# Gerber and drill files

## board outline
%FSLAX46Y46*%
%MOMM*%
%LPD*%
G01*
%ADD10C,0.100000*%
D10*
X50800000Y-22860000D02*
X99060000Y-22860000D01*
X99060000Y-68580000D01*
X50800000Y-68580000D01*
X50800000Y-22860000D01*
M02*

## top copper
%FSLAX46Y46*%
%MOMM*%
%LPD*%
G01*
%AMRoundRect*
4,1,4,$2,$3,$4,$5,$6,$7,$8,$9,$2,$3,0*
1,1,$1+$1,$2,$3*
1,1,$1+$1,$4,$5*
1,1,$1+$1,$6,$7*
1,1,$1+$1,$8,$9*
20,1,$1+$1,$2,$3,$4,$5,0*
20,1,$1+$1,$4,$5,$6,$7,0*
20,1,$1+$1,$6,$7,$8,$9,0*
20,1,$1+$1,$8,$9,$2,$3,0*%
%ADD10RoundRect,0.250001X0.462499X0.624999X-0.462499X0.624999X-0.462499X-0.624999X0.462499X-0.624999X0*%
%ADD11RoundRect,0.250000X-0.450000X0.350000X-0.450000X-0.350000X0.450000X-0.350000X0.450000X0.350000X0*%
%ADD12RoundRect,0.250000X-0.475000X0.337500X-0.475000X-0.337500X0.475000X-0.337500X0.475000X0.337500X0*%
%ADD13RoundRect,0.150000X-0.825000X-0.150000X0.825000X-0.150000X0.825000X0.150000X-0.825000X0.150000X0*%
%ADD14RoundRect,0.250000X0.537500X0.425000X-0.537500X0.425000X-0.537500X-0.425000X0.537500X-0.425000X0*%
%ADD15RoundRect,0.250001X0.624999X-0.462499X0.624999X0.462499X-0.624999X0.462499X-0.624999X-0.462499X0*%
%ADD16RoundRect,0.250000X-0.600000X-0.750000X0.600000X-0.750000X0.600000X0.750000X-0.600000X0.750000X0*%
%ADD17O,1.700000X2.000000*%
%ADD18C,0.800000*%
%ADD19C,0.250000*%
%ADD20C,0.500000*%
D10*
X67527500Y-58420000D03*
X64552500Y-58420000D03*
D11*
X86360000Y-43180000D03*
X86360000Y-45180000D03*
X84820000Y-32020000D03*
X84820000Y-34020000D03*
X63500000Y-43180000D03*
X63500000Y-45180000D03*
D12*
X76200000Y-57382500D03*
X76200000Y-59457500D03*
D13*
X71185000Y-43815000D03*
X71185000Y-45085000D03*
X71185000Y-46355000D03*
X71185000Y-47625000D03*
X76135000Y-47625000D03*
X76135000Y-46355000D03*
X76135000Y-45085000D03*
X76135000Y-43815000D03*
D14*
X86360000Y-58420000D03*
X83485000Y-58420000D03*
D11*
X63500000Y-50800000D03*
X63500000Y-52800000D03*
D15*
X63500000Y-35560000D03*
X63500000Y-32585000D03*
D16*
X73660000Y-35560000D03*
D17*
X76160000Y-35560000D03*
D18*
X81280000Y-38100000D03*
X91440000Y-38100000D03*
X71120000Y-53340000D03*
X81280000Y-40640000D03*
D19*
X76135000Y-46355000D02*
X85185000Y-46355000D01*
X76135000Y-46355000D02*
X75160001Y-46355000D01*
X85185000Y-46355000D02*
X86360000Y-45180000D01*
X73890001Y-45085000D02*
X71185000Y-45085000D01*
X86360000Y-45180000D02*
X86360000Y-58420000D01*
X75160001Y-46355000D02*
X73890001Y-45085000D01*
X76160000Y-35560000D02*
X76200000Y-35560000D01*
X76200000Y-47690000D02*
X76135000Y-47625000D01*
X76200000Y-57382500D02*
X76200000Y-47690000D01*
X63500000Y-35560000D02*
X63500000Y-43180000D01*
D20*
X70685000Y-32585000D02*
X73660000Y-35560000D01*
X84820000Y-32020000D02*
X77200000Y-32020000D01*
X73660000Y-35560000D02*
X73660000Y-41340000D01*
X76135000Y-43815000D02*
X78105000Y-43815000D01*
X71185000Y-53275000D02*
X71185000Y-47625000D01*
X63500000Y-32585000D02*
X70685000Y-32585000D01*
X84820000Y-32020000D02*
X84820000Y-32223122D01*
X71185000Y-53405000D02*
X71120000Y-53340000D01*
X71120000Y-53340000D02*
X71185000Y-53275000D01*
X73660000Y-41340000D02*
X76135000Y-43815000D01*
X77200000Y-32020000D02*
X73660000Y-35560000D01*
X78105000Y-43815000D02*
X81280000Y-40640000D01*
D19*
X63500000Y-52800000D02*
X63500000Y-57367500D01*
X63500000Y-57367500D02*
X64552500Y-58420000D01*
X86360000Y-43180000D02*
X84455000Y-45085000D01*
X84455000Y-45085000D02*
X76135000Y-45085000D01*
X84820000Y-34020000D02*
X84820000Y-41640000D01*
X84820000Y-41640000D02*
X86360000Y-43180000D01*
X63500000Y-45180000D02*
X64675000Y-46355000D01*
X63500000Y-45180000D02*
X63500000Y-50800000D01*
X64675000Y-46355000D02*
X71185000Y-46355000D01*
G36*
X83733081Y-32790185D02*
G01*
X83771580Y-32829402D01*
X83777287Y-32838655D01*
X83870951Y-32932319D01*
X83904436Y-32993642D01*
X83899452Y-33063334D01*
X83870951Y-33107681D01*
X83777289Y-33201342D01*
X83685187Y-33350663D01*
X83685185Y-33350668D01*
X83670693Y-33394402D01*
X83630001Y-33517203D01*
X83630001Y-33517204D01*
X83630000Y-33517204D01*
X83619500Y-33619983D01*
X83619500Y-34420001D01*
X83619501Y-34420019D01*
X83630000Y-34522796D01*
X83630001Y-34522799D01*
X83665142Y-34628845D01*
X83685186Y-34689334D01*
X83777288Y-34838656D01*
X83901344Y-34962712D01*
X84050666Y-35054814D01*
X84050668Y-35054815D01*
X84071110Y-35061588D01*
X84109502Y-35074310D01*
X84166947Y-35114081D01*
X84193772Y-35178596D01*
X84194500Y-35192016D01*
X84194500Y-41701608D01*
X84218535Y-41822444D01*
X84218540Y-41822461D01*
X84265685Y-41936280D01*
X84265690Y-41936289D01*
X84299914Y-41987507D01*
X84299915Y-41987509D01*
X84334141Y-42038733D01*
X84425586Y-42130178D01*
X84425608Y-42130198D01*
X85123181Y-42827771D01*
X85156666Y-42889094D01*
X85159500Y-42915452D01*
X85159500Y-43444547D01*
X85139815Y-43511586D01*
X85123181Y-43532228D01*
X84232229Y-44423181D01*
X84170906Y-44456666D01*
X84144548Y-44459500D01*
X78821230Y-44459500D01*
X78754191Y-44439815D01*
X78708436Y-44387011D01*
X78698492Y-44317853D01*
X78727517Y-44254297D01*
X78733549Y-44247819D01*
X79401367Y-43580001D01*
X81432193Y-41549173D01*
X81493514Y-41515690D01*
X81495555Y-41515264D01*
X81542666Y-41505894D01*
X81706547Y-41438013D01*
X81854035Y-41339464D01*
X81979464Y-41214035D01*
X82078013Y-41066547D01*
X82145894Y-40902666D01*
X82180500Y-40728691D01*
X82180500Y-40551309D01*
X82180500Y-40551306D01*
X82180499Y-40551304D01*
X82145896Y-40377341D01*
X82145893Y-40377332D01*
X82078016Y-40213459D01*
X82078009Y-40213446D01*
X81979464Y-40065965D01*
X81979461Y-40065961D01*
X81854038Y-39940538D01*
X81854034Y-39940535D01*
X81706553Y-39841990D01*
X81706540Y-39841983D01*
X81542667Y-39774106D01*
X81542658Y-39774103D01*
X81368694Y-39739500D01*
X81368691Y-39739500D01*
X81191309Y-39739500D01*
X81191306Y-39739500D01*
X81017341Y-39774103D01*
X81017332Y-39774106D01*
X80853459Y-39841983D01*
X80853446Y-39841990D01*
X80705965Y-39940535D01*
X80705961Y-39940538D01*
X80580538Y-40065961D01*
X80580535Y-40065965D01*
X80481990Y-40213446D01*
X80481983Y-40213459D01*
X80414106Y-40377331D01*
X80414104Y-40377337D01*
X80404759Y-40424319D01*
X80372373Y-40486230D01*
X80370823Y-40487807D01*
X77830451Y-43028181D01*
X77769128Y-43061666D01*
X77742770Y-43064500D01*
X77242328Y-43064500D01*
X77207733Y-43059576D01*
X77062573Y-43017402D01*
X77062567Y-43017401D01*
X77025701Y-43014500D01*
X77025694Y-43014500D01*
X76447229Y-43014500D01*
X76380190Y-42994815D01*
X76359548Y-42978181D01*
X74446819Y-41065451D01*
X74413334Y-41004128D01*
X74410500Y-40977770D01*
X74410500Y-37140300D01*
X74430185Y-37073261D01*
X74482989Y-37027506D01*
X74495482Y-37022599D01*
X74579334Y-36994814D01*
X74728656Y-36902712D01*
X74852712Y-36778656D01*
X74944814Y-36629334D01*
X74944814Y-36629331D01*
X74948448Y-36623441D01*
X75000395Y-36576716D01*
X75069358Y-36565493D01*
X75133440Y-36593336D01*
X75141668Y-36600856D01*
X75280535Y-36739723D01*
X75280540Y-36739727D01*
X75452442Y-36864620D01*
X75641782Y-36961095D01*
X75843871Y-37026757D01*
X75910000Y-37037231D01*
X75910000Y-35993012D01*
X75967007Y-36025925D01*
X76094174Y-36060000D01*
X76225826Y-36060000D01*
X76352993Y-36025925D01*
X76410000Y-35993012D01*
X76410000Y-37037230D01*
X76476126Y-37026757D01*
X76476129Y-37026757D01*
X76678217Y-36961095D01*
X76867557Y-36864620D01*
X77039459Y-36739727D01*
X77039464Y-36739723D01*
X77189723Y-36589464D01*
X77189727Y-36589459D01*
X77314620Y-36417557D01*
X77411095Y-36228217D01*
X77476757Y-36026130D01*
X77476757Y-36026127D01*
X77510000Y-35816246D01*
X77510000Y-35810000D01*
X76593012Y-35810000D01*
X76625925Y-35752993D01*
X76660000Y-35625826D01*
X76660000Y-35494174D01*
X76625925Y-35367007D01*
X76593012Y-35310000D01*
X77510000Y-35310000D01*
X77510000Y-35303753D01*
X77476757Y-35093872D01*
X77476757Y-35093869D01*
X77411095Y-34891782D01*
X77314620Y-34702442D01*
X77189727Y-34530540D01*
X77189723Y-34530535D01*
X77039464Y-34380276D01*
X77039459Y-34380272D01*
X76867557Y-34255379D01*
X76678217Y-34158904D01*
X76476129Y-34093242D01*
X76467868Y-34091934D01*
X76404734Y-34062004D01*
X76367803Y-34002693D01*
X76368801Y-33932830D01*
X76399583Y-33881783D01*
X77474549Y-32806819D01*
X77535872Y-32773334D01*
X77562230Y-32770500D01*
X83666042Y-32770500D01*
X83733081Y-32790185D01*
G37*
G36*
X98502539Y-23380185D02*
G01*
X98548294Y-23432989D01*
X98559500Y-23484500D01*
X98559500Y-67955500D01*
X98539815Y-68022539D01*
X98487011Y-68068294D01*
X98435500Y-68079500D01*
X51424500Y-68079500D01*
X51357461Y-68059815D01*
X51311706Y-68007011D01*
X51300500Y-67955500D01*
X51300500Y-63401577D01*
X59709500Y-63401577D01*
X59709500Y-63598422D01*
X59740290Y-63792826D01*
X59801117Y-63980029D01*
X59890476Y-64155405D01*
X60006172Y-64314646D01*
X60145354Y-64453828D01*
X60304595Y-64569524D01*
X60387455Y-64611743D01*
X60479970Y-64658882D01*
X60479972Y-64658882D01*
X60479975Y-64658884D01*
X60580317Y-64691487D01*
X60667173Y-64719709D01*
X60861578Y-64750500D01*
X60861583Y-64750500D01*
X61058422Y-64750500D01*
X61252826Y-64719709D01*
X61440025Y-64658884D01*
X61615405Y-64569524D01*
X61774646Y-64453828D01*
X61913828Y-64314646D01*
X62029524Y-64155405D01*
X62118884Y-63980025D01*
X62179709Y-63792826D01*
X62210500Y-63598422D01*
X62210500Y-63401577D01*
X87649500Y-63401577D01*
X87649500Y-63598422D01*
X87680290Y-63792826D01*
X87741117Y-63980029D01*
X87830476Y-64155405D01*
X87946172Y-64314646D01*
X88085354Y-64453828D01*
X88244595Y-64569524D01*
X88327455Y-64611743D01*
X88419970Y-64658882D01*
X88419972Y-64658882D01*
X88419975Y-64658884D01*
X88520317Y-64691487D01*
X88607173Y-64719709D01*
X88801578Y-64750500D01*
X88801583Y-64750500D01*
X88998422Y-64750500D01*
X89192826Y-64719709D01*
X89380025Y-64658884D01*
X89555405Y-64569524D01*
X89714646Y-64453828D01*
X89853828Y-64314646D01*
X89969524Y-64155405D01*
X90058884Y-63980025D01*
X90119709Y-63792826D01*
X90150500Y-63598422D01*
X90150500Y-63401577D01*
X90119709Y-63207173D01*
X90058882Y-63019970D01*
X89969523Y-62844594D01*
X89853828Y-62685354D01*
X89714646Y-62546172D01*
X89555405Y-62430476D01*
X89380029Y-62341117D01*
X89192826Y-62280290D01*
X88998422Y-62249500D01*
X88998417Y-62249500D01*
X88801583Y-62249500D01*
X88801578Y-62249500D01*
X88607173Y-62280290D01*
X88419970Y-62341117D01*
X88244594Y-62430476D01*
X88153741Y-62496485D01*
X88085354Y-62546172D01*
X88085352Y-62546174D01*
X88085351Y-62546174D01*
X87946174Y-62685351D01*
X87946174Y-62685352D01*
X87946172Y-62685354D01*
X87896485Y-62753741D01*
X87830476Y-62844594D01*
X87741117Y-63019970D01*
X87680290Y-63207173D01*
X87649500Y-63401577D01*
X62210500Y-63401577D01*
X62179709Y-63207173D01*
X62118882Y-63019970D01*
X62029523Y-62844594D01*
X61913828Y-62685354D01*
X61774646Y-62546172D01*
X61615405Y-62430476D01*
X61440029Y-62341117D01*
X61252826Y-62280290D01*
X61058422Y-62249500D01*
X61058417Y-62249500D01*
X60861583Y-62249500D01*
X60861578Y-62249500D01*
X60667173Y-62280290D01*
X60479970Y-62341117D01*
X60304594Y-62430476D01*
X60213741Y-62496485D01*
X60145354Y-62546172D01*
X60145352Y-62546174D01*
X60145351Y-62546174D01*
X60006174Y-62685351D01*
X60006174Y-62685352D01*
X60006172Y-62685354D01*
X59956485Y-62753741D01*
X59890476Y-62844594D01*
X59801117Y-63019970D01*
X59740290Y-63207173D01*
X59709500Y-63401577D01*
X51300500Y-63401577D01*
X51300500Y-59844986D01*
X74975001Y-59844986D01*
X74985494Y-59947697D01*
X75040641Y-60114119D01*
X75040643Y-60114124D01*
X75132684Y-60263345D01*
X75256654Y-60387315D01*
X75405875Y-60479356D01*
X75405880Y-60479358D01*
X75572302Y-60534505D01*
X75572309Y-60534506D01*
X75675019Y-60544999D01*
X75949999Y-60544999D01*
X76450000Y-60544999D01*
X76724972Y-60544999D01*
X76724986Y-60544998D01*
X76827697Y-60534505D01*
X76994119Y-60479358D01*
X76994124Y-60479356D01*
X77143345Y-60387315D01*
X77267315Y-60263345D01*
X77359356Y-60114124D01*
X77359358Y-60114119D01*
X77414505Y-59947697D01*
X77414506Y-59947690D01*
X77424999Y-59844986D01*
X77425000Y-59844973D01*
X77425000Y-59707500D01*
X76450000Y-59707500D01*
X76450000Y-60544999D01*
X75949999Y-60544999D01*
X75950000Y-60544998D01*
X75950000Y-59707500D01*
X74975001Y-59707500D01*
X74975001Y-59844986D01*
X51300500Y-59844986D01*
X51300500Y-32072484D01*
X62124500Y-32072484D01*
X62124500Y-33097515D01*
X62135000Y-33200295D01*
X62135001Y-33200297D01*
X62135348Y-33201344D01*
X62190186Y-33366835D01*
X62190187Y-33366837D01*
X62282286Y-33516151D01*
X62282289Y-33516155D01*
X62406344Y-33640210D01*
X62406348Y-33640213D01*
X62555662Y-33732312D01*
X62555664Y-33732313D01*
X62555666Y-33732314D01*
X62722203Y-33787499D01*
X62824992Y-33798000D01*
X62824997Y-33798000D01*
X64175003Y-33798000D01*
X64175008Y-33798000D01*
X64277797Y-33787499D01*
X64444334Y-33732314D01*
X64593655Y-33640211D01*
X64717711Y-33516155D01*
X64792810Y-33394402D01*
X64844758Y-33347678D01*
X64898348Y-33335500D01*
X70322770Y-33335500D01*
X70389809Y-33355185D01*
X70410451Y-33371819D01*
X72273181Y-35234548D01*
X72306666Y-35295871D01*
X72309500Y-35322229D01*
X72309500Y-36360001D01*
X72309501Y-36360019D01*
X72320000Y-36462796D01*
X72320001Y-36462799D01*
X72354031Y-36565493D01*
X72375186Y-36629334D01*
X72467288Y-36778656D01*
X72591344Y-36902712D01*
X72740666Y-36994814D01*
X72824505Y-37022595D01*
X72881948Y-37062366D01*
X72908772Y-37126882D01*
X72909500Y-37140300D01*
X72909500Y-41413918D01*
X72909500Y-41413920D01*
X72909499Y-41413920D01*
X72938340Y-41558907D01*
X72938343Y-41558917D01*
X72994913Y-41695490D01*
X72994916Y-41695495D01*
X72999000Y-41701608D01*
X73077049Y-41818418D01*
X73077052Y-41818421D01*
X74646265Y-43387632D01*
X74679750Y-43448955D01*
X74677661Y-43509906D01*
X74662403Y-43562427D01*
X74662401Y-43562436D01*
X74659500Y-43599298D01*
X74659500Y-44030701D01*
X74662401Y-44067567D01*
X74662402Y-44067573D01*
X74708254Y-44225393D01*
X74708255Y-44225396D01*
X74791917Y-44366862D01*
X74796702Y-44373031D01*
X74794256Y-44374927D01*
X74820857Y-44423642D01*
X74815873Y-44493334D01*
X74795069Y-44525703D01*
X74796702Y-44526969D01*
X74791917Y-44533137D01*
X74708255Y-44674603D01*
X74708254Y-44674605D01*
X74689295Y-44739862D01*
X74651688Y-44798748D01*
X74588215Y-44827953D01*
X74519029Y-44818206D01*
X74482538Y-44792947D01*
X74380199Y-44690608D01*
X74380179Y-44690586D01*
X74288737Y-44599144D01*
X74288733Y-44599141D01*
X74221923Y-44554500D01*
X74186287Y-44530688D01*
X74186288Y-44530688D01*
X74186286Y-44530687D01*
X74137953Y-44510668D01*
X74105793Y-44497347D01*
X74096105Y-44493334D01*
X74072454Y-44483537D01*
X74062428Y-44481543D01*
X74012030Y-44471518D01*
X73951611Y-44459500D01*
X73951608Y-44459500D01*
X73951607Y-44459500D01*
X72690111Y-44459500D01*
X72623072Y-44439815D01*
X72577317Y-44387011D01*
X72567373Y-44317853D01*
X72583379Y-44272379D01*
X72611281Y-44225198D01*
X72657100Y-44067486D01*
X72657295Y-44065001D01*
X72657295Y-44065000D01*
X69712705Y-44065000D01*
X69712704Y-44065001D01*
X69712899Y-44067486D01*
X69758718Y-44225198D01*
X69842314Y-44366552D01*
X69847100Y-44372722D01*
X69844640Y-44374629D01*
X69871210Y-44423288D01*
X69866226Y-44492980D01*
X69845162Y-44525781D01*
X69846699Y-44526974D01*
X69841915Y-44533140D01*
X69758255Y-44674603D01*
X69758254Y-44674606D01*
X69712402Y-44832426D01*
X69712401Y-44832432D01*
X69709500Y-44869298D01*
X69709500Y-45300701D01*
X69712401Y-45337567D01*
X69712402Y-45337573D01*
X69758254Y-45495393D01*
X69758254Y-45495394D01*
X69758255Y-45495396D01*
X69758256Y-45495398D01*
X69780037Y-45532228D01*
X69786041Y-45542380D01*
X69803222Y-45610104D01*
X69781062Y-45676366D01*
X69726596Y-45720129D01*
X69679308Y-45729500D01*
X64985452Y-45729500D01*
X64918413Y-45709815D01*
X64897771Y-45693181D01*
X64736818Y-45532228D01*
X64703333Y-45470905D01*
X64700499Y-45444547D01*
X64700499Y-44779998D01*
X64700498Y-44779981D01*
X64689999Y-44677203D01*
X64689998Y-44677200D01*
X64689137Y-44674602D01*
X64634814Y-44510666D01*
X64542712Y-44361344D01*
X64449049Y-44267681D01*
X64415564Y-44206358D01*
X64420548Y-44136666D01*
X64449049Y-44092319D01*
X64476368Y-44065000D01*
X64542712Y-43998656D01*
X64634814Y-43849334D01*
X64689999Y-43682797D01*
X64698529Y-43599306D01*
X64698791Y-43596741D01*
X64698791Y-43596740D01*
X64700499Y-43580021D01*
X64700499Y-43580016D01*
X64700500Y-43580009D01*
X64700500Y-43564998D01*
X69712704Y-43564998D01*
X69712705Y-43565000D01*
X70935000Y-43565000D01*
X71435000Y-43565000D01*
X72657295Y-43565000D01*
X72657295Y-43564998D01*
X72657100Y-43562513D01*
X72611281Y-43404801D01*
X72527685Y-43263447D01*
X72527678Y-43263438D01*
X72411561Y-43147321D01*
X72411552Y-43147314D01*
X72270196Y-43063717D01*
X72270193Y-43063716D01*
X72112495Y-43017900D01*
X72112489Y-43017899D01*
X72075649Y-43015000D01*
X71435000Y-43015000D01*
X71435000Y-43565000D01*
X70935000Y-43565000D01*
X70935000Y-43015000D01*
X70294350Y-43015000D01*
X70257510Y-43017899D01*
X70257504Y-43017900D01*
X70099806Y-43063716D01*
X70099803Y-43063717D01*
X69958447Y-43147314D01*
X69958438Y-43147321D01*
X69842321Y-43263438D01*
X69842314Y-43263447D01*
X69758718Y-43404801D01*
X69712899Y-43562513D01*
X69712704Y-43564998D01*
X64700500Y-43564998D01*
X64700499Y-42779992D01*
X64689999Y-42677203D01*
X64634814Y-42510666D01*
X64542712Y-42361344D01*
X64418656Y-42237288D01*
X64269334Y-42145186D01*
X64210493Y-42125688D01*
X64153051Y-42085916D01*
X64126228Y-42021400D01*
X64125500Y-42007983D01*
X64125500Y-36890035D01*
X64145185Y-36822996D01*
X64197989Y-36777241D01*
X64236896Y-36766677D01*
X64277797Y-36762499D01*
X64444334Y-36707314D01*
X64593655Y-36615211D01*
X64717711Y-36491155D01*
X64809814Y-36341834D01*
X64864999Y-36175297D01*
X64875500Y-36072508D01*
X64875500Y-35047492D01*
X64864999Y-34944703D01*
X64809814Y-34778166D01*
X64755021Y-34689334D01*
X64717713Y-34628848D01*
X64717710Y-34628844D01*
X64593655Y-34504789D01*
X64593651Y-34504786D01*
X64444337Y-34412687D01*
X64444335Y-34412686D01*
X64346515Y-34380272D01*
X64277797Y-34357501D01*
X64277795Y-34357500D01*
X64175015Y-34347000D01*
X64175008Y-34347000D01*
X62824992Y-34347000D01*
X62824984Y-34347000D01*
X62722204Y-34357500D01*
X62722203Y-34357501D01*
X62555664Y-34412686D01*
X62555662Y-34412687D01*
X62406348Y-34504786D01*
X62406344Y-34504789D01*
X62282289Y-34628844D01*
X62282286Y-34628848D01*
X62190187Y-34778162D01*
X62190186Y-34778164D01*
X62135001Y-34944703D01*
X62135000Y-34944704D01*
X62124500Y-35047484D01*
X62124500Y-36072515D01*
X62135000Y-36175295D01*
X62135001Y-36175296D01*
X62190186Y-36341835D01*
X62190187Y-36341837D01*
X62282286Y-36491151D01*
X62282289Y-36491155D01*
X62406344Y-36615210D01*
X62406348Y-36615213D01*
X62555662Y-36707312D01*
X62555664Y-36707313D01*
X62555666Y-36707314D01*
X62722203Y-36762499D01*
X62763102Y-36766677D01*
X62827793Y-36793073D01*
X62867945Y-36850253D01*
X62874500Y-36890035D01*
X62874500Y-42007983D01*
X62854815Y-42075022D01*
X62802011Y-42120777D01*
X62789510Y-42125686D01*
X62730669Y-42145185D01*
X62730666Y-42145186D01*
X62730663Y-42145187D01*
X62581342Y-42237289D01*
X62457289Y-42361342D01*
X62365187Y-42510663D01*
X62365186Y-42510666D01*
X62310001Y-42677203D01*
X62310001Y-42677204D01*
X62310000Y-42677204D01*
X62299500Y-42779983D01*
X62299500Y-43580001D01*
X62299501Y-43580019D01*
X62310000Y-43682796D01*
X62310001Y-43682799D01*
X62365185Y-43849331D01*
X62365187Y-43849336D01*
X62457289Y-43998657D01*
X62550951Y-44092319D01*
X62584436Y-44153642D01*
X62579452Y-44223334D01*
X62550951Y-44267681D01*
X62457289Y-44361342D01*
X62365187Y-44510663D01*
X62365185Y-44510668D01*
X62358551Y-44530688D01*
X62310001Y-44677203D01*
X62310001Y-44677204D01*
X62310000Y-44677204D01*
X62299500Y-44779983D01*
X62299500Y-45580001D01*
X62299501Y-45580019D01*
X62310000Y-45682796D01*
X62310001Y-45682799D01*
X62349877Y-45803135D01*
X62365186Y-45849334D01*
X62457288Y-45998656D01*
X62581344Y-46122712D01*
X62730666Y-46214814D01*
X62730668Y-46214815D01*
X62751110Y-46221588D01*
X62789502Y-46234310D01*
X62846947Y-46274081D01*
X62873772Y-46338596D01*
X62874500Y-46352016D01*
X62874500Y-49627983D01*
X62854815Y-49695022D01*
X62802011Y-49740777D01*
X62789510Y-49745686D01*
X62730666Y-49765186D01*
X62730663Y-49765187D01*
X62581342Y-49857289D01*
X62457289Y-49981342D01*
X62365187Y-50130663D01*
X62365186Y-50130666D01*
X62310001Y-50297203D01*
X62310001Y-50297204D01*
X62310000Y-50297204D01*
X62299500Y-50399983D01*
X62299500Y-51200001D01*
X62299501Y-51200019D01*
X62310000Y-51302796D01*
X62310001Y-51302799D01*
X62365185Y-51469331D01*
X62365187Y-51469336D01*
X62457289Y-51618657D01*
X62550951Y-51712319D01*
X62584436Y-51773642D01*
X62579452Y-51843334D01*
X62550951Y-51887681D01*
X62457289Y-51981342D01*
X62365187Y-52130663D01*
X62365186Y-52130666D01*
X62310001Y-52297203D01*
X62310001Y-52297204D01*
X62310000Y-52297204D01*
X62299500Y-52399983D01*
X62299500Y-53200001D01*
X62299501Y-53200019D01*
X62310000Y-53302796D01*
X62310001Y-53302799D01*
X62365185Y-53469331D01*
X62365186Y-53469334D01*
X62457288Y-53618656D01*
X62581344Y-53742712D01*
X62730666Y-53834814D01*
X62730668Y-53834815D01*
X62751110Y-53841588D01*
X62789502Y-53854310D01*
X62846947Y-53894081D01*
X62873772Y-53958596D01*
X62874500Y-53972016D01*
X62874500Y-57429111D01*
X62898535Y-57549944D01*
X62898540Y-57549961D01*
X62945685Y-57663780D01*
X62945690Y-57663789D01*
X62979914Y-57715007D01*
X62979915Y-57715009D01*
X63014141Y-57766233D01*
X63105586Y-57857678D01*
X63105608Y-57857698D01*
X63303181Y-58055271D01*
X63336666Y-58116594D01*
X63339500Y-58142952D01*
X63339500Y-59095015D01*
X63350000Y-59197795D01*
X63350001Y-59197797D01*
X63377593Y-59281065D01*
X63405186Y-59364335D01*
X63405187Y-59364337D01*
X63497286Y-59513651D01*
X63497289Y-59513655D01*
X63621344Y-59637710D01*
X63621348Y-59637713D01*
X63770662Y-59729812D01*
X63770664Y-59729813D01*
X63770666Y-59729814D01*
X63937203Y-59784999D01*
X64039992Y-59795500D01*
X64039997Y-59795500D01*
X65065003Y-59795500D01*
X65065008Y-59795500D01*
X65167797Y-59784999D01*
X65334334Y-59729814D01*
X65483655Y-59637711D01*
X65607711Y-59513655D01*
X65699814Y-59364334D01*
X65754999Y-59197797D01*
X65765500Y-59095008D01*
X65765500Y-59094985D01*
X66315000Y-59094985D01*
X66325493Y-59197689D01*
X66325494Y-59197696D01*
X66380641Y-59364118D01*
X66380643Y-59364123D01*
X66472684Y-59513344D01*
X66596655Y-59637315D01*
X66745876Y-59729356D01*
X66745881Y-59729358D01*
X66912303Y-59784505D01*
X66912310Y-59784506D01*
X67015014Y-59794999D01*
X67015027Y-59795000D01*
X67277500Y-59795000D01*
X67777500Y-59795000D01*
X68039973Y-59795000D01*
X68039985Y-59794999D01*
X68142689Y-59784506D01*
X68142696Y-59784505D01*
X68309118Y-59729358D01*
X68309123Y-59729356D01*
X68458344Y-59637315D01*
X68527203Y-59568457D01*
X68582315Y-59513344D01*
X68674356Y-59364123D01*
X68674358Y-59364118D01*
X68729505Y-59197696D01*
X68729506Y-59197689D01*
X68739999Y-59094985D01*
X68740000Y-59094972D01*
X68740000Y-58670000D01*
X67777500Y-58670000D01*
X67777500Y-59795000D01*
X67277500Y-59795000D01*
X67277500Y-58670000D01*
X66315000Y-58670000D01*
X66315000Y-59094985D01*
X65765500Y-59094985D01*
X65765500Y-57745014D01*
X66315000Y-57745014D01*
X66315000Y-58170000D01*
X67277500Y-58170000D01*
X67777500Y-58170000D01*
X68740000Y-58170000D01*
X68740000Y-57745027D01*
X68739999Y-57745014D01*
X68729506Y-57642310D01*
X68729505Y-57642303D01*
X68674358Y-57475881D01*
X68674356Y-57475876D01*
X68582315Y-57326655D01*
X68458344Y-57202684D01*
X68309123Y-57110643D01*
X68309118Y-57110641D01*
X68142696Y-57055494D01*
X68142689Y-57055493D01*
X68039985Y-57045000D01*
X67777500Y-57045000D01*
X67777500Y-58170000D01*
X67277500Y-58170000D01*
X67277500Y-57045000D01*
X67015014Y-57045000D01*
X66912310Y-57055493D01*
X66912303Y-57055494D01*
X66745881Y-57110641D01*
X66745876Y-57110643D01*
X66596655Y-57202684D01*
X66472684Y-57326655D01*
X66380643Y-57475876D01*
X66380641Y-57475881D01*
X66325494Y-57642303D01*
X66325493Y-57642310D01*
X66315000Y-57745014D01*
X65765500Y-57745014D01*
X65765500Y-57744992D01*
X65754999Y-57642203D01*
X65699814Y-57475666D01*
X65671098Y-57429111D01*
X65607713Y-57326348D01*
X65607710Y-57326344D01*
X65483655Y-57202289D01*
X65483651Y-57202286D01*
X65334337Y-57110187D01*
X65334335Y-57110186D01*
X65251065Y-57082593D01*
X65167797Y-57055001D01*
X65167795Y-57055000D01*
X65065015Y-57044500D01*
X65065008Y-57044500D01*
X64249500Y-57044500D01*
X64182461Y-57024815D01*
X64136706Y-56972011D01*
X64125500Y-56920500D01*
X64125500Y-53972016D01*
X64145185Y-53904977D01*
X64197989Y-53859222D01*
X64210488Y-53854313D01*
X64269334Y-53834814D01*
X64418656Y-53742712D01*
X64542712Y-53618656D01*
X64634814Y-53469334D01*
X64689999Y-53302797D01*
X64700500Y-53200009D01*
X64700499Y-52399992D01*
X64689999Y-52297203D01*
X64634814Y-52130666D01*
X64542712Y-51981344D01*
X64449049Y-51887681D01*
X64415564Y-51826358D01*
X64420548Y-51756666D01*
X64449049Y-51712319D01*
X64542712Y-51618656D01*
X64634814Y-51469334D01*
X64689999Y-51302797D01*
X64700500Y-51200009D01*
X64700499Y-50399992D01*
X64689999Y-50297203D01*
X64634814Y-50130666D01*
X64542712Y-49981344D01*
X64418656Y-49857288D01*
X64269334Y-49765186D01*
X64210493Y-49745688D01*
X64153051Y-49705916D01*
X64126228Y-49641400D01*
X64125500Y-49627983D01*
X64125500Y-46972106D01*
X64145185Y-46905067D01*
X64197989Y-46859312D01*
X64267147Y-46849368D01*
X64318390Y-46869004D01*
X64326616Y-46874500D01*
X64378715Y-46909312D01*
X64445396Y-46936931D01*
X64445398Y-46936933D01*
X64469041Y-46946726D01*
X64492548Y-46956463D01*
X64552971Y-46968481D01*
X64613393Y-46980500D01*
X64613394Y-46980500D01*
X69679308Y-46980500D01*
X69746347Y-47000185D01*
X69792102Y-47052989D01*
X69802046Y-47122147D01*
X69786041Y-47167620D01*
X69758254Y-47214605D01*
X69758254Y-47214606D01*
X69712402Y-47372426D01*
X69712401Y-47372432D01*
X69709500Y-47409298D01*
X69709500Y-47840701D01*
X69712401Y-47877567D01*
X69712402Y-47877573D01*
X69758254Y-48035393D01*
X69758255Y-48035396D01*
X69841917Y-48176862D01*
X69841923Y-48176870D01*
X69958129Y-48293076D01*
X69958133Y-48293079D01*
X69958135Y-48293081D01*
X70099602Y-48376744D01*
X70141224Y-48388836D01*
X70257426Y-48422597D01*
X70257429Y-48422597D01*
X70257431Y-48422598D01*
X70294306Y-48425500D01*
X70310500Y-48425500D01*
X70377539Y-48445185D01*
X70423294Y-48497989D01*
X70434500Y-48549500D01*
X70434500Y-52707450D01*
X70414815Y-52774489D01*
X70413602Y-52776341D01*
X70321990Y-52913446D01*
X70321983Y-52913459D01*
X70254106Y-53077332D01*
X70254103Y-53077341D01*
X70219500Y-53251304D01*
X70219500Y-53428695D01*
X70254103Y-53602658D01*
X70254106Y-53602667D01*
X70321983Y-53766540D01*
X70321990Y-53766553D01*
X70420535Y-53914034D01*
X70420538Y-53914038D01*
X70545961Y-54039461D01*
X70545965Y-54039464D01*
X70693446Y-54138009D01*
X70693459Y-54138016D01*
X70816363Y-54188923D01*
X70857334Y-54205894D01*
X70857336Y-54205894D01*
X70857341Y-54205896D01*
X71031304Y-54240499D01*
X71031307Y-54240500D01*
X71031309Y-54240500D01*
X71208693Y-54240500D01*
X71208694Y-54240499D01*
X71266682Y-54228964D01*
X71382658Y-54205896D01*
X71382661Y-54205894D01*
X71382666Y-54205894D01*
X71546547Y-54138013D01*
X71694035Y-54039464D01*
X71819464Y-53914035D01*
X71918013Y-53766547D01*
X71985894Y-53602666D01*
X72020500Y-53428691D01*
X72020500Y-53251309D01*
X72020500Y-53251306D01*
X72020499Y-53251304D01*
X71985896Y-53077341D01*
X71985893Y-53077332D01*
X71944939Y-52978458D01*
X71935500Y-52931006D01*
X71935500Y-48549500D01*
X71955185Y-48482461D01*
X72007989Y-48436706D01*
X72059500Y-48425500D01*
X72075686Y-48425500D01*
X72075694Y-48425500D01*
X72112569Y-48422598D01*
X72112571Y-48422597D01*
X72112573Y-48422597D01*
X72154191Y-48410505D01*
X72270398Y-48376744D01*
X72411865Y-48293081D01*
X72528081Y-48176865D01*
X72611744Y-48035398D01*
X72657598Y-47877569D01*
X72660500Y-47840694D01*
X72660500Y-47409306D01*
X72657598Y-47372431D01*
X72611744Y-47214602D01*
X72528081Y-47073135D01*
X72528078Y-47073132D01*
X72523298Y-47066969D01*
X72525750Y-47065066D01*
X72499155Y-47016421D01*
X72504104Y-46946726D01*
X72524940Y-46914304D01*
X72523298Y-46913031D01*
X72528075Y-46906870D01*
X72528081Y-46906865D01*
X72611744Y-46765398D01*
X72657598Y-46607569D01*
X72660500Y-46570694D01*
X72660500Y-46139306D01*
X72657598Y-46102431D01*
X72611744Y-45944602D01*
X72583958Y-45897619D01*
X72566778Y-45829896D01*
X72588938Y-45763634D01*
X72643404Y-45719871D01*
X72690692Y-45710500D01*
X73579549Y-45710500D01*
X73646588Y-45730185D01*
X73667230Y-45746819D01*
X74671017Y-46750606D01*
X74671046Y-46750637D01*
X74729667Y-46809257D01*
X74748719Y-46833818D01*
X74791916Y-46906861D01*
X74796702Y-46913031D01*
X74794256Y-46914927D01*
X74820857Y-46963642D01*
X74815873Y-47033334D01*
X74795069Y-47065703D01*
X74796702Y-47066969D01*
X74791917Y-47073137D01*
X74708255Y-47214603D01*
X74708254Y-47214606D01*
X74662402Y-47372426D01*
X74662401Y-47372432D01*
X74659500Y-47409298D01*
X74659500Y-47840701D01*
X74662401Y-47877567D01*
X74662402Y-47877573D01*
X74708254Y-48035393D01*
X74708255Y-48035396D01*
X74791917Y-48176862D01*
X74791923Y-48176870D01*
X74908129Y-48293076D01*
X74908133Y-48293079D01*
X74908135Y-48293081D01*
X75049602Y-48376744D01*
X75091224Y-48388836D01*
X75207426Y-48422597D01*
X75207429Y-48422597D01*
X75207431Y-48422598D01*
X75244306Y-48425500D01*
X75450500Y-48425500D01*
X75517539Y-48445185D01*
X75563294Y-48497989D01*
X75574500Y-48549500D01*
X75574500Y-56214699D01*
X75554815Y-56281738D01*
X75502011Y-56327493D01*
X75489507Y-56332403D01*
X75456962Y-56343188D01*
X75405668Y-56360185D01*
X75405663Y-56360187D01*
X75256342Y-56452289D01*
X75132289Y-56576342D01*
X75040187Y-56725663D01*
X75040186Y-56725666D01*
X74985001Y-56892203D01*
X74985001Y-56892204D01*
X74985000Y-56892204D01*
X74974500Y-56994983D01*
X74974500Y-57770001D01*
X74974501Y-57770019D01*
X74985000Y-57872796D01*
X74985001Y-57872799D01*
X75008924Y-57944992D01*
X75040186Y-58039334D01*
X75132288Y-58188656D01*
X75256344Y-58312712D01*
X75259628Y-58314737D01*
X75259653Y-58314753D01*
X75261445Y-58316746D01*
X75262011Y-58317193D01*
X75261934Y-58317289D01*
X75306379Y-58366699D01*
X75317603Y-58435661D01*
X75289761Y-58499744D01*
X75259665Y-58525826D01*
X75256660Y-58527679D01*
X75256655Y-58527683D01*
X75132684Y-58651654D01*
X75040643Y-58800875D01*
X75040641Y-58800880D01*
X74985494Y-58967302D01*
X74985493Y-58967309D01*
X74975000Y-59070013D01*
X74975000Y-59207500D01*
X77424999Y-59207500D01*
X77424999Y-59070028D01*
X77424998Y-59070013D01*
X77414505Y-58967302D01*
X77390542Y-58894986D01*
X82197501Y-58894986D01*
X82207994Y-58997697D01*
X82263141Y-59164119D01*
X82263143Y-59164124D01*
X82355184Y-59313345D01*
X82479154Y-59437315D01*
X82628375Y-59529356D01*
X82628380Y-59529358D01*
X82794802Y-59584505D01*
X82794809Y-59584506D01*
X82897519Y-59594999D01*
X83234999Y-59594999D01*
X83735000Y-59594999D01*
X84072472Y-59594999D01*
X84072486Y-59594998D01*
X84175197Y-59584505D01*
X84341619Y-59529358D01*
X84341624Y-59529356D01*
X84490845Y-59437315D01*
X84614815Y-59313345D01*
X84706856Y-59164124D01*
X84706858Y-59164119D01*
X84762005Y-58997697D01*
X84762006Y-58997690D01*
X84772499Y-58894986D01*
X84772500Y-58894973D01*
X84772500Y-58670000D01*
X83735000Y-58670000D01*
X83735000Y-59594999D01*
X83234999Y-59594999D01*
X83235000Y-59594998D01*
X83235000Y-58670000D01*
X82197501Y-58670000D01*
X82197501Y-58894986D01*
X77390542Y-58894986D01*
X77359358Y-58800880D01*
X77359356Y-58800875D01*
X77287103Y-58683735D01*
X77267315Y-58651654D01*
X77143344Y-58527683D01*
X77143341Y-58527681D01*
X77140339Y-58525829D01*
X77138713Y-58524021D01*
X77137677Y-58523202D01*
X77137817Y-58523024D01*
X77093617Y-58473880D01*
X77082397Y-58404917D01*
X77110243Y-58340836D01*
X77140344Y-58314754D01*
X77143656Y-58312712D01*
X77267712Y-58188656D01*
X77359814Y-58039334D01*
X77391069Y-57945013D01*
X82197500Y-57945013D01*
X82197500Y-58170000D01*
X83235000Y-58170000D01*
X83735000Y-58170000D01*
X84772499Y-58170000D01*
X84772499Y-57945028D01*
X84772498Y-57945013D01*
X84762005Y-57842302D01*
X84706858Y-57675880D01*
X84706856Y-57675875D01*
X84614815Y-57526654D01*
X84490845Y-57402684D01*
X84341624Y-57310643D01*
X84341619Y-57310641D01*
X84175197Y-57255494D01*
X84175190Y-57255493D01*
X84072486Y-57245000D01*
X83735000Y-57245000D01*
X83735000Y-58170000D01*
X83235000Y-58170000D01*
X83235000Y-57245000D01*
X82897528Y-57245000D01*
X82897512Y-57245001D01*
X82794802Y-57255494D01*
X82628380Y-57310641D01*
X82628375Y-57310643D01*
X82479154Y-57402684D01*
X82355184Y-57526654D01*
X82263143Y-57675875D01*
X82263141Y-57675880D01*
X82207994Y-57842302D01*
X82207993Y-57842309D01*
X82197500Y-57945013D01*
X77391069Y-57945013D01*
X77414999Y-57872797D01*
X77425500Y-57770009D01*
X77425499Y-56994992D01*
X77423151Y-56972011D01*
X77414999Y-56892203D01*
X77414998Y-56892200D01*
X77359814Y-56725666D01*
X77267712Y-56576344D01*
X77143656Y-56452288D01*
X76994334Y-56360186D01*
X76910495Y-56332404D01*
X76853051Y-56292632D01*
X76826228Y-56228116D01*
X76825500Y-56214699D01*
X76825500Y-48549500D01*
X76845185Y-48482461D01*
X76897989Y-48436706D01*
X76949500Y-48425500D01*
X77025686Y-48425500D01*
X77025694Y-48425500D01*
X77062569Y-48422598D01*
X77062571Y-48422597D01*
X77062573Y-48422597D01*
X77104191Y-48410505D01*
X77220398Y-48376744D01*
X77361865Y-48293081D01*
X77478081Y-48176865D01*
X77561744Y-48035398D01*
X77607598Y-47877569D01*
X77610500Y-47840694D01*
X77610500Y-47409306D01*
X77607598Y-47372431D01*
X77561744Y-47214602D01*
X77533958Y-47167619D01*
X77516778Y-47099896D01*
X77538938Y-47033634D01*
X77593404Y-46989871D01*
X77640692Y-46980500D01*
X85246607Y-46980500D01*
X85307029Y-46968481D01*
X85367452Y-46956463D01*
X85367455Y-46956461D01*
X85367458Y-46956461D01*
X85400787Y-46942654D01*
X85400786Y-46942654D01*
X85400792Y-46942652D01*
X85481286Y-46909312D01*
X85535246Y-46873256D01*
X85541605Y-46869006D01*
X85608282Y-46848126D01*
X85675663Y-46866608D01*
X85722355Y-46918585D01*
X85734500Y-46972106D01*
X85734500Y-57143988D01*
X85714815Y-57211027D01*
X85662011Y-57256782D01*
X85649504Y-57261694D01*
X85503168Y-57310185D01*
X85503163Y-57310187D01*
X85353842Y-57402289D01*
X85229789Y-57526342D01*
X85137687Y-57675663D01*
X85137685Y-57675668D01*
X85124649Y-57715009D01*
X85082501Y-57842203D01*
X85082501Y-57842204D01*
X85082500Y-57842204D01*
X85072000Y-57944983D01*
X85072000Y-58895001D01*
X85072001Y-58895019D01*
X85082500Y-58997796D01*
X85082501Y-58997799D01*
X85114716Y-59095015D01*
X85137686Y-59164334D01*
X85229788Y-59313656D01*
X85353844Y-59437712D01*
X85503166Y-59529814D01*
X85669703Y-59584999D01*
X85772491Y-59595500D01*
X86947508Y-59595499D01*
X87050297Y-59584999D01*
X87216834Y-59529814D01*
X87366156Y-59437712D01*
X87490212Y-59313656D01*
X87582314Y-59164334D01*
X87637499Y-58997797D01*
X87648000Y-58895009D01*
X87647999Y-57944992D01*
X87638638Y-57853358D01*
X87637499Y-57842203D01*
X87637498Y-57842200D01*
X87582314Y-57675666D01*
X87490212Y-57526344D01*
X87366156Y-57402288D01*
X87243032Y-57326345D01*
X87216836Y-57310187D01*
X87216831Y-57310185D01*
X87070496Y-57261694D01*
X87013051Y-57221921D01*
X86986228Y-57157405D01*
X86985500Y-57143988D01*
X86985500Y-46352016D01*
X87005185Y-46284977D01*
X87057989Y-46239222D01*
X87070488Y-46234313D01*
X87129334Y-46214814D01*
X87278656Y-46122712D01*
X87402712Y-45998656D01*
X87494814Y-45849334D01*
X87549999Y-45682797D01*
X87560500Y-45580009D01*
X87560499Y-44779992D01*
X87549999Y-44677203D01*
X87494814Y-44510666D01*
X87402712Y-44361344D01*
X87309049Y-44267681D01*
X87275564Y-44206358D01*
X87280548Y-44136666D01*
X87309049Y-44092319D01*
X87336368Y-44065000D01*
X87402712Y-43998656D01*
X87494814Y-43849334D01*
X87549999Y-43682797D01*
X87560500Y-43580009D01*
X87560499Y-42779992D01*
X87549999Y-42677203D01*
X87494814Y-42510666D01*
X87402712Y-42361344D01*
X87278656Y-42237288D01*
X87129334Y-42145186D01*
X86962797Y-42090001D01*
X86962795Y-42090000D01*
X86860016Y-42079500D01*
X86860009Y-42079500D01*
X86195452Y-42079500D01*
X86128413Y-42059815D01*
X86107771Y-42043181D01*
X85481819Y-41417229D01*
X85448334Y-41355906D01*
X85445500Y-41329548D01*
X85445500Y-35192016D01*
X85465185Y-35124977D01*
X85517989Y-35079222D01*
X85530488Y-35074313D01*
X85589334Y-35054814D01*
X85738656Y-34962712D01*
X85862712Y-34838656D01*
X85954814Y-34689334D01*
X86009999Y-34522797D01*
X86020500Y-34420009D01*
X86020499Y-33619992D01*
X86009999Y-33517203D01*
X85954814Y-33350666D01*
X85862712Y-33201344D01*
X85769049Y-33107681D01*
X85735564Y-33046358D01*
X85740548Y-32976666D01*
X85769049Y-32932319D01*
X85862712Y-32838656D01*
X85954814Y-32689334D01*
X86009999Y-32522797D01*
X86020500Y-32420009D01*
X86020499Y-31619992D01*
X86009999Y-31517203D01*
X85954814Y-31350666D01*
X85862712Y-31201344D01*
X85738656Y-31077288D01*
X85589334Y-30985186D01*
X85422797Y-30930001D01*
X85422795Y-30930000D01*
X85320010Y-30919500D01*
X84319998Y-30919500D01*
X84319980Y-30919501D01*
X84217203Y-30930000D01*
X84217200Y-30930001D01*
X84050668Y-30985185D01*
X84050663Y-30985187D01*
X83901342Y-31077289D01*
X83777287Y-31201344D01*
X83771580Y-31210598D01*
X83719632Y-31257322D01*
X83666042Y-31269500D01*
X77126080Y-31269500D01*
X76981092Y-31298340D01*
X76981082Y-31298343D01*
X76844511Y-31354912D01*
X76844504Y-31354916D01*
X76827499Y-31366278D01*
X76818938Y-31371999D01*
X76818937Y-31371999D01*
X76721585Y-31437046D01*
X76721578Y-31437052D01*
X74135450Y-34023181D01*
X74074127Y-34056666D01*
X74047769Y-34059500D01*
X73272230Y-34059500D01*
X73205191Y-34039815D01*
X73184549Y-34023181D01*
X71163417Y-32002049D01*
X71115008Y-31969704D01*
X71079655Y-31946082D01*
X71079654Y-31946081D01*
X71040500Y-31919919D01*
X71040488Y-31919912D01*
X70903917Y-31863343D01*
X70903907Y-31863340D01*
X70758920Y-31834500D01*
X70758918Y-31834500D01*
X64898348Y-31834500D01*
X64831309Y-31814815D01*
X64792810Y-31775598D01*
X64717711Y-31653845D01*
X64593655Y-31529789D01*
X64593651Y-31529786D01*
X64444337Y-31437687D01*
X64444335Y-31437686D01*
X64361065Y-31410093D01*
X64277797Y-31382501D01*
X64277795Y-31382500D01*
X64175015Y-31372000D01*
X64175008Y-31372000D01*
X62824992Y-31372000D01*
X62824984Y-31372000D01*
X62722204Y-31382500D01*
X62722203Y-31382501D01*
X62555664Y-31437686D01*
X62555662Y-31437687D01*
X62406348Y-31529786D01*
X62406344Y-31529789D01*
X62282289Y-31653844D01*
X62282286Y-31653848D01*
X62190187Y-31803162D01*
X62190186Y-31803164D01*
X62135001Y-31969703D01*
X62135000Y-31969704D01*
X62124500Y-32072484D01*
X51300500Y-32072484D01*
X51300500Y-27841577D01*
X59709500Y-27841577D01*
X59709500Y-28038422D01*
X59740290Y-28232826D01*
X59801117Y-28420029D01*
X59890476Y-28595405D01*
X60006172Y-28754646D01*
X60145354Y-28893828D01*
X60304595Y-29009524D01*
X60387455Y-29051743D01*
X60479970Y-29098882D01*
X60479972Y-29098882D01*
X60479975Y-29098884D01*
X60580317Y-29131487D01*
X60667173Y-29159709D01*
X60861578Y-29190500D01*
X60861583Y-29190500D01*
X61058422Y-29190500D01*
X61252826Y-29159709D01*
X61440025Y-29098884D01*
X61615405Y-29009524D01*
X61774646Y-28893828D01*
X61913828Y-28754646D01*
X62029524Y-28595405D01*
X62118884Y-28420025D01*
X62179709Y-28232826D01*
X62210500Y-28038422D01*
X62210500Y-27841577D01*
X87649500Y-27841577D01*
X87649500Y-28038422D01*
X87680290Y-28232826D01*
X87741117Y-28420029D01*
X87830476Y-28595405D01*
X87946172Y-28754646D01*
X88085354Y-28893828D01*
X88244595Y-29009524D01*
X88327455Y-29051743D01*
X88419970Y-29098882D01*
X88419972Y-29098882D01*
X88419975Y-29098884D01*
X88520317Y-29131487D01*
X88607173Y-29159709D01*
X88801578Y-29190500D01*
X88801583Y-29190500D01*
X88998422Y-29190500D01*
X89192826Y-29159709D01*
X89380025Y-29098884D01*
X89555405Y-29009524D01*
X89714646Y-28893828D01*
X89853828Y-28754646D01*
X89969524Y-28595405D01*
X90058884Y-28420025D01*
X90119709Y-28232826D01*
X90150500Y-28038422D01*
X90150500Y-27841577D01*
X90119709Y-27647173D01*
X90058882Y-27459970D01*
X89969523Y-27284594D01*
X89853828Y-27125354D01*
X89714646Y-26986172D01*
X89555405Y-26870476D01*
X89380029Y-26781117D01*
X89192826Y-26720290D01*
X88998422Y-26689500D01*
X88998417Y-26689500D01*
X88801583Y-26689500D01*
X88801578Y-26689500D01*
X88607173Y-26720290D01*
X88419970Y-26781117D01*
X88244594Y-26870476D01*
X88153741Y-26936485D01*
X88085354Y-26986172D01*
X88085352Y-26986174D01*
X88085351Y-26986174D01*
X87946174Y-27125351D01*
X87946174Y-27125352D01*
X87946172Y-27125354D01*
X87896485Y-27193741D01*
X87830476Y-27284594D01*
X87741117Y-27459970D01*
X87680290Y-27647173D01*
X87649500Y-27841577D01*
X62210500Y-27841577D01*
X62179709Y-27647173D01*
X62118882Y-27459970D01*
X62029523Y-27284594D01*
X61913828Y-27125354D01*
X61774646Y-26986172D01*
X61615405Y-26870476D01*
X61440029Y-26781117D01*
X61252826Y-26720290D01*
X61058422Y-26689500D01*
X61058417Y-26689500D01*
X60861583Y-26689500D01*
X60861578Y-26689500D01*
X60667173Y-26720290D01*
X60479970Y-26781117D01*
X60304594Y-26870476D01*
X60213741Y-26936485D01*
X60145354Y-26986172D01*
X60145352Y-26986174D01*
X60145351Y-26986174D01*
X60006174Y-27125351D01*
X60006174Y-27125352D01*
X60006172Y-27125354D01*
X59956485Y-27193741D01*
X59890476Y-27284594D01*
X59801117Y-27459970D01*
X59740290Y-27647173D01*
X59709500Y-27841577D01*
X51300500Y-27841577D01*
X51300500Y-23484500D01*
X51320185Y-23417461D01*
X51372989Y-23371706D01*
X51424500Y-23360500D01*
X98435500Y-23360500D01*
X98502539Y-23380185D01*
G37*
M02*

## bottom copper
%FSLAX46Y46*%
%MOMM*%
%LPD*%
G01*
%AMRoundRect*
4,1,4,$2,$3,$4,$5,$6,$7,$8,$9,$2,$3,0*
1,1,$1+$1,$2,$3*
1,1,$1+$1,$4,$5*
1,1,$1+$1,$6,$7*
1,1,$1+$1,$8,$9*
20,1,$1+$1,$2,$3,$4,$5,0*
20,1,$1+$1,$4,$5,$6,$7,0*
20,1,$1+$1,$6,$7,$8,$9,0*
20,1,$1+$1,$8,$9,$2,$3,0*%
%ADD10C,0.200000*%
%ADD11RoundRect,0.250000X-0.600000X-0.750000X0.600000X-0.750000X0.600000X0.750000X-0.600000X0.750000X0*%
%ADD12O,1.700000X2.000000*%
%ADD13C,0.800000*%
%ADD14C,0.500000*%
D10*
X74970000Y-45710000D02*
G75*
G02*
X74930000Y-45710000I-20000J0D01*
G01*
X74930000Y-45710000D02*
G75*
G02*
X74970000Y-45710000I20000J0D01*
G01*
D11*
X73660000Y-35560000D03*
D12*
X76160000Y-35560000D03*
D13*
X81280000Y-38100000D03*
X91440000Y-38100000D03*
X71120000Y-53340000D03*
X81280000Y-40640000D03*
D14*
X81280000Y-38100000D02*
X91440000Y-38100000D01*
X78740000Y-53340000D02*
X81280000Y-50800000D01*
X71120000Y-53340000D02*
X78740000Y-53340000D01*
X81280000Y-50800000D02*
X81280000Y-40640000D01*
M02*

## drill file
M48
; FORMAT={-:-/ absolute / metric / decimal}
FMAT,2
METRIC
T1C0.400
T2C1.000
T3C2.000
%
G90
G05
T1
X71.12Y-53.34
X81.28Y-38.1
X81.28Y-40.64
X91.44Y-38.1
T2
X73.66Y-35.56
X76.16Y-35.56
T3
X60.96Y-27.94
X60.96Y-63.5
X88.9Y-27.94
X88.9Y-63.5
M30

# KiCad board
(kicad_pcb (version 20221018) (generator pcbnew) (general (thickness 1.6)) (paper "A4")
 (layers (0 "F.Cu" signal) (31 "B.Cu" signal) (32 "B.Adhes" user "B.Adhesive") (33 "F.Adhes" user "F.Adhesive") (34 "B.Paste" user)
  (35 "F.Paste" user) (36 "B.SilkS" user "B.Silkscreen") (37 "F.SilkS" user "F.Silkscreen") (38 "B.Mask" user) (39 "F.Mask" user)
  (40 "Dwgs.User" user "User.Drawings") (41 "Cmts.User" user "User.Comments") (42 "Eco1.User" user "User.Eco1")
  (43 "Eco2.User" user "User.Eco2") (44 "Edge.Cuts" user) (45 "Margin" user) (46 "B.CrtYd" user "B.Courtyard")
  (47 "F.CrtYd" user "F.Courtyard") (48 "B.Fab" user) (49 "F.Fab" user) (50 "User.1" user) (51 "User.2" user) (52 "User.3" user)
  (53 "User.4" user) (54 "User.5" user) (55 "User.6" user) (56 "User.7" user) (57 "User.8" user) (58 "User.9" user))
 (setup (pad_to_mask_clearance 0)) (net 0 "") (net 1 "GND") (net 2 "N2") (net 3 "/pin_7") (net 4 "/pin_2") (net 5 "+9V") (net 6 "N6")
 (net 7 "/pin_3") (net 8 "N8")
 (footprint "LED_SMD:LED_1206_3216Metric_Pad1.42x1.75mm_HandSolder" (layer "F.Cu") (at 66.04 58.42 180)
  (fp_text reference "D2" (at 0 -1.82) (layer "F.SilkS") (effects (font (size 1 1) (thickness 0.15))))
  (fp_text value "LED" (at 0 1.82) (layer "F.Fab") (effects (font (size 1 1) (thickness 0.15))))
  (pad "1" smd roundrect (at -1.4875 0 180) (size 1.425 1.75) (layers "F.Cu" "F.Paste" "F.Mask") (roundrect_rratio 0.1754392982)
   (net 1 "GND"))
  (pad "2" smd roundrect (at 1.4875 0 180) (size 1.425 1.75) (layers "F.Cu" "F.Paste" "F.Mask") (roundrect_rratio 0.1754392982) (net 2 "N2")))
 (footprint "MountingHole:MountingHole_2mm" (layer "F.Cu") (at 60.96 63.5)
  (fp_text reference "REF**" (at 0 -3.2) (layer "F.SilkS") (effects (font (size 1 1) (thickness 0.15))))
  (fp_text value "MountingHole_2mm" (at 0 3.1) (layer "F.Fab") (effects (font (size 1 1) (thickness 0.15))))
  (pad "" np_thru_hole circle (at 0 0) (size 2 2) (drill 2) (layers "*.Cu" "*.Mask")))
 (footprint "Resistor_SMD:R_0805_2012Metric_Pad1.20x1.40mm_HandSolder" (layer "F.Cu") (at 86.36 44.18 -90)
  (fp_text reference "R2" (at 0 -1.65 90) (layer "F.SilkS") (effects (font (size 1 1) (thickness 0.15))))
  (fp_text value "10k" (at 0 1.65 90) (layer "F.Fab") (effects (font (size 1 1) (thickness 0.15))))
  (pad "1" smd roundrect (at -1 0 270) (size 1.2 1.4) (layers "F.Cu" "F.Paste" "F.Mask") (roundrect_rratio 0.2083333333) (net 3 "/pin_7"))
  (pad "2" smd roundrect (at 1 0 270) (size 1.2 1.4) (layers "F.Cu" "F.Paste" "F.Mask") (roundrect_rratio 0.2083333333) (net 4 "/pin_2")))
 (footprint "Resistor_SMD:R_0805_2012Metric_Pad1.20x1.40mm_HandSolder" (layer "F.Cu") (at 84.82 33.02 -90)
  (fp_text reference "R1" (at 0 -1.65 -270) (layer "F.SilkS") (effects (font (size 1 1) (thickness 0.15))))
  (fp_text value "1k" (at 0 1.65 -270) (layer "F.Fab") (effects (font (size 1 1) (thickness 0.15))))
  (pad "1" smd roundrect (at -1 0 270) (size 1.2 1.4) (layers "F.Cu" "F.Paste" "F.Mask") (roundrect_rratio 0.2083333333) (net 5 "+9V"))
  (pad "2" smd roundrect (at 1 0 270) (size 1.2 1.4) (layers "F.Cu" "F.Paste" "F.Mask") (roundrect_rratio 0.2083333333) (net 3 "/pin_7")))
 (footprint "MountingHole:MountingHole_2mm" (layer "F.Cu") (at 88.9 63.5)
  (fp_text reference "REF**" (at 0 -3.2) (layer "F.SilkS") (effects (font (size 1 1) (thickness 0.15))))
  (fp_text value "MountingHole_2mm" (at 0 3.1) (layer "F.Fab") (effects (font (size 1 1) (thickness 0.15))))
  (pad "" np_thru_hole circle (at 0 0) (size 2 2) (drill 2) (layers "*.Cu" "*.Mask")))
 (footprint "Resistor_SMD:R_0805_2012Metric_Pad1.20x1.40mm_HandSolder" (layer "F.Cu") (at 63.5 44.18 -90)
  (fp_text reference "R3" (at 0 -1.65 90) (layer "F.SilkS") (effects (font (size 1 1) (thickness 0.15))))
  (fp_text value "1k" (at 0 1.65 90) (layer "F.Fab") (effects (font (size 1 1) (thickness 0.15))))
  (pad "1" smd roundrect (at -1 0 270) (size 1.2 1.4) (layers "F.Cu" "F.Paste" "F.Mask") (roundrect_rratio 0.2083333333) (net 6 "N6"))
  (pad "2" smd roundrect (at 1 0 270) (size 1.2 1.4) (layers "F.Cu" "F.Paste" "F.Mask") (roundrect_rratio 0.2083333333) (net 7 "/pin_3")))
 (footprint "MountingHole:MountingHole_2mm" (layer "F.Cu") (at 88.9 27.94)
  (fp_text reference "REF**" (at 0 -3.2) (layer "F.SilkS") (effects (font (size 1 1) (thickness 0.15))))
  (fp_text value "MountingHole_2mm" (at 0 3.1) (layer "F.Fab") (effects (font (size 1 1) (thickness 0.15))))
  (pad "" np_thru_hole circle (at 0 0) (size 2 2) (drill 2) (layers "*.Cu" "*.Mask")))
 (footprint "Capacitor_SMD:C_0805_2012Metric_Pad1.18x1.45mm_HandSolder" (layer "F.Cu") (at 76.2 58.42 -90)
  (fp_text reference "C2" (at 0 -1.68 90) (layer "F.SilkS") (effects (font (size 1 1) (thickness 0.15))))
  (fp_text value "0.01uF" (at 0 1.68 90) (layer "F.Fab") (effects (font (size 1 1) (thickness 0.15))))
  (pad "1" smd roundrect (at -1.0375 0 270) (size 1.175 1.45) (layers "F.Cu" "F.Paste" "F.Mask") (roundrect_rratio 0.2127659574)
   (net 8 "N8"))
  (pad "2" smd roundrect (at 1.0375 0 270) (size 1.175 1.45) (layers "F.Cu" "F.Paste" "F.Mask") (roundrect_rratio 0.2127659574)
   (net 1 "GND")))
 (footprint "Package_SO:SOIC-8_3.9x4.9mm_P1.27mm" (layer "F.Cu") (at 73.66 45.72)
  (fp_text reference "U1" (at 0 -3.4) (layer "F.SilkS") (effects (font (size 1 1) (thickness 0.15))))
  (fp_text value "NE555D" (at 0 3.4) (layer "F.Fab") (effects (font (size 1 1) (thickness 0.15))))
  (pad "1" smd roundrect (at -2.475 -1.905) (size 1.95 0.6) (layers "F.Cu" "F.Paste" "F.Mask") (roundrect_rratio 0.25) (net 1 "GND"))
  (pad "2" smd roundrect (at -2.475 -0.635) (size 1.95 0.6) (layers "F.Cu" "F.Paste" "F.Mask") (roundrect_rratio 0.25) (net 4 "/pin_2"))
  (pad "3" smd roundrect (at -2.475 0.635) (size 1.95 0.6) (layers "F.Cu" "F.Paste" "F.Mask") (roundrect_rratio 0.25) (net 7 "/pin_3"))
  (pad "4" smd roundrect (at -2.475 1.905) (size 1.95 0.6) (layers "F.Cu" "F.Paste" "F.Mask") (roundrect_rratio 0.25) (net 5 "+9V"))
  (pad "5" smd roundrect (at 2.475 1.905) (size 1.95 0.6) (layers "F.Cu" "F.Paste" "F.Mask") (roundrect_rratio 0.25) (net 8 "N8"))
  (pad "6" smd roundrect (at 2.475 0.635) (size 1.95 0.6) (layers "F.Cu" "F.Paste" "F.Mask") (roundrect_rratio 0.25) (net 4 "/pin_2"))
  (pad "7" smd roundrect (at 2.475 -0.635) (size 1.95 0.6) (layers "F.Cu" "F.Paste" "F.Mask") (roundrect_rratio 0.25) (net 3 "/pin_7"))
  (pad "8" smd roundrect (at 2.475 -1.905) (size 1.95 0.6) (layers "F.Cu" "F.Paste" "F.Mask") (roundrect_rratio 0.25) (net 5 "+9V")))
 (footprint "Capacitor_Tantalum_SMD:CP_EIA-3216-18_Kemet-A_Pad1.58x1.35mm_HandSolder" (layer "F.Cu") (at 84.9225 58.42 180)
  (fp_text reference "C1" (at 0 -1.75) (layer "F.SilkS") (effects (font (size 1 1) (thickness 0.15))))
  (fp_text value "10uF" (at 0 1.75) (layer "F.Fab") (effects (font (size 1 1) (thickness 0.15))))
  (pad "1" smd roundrect (at -1.4375 0 180) (size 1.575 1.35) (layers "F.Cu" "F.Paste" "F.Mask") (roundrect_rratio 0.1851851852)
   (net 4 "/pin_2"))
  (pad "2" smd roundrect (at 1.4375 0 180) (size 1.575 1.35) (layers "F.Cu" "F.Paste" "F.Mask") (roundrect_rratio 0.1851851852)
   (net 1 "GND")))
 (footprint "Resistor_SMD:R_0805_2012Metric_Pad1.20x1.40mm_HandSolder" (layer "F.Cu") (at 63.5 51.8 -90)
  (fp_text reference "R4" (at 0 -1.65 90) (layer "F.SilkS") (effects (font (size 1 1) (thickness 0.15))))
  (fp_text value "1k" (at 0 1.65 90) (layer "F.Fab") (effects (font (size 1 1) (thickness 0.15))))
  (pad "1" smd roundrect (at -1 0 270) (size 1.2 1.4) (layers "F.Cu" "F.Paste" "F.Mask") (roundrect_rratio 0.2083333333) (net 7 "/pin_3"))
  (pad "2" smd roundrect (at 1 0 270) (size 1.2 1.4) (layers "F.Cu" "F.Paste" "F.Mask") (roundrect_rratio 0.2083333333) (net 2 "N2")))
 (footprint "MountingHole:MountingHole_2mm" (layer "F.Cu") (at 60.96 27.94)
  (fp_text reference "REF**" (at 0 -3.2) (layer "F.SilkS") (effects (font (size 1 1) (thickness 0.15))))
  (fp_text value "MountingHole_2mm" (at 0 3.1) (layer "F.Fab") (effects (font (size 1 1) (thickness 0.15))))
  (pad "" np_thru_hole circle (at 0 0) (size 2 2) (drill 2) (layers "*.Cu" "*.Mask")))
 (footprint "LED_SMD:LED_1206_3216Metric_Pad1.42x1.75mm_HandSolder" (layer "F.Cu") (at 63.5 34.0725 90)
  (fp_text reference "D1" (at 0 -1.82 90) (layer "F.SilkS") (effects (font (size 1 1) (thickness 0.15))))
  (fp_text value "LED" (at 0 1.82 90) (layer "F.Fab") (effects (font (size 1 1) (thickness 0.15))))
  (pad "1" smd roundrect (at -1.4875 0 90) (size 1.425 1.75) (layers "F.Cu" "F.Paste" "F.Mask") (roundrect_rratio 0.1754392982) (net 6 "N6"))
  (pad "2" smd roundrect (at 1.4875 0 90) (size 1.425 1.75) (layers "F.Cu" "F.Paste" "F.Mask") (roundrect_rratio 0.1754392982) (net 5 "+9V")))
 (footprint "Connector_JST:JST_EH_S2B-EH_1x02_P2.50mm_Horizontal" (layer "F.Cu") (at 73.66 35.56)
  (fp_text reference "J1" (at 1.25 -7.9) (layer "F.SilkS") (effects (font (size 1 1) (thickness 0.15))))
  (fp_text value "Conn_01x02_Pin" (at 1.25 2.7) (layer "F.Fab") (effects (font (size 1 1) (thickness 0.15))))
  (pad "1" thru_hole roundrect (at 0 0) (size 1.7 2) (drill 1) (layers "*.Cu" "*.Mask") (roundrect_rratio 0.1470588235) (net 5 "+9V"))
  (pad "2" thru_hole oval (at 2.5 0) (size 1.7 2) (drill 1) (layers "*.Cu" "*.Mask") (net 1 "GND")))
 (gr_circle (center 74.95 45.71) (end 74.95 45.69) (stroke (width 0.2) (type default)) (fill none) (layer "B.Cu"))
 (gr_rect (start 50.8 22.86) (end 99.06 68.58) (stroke (width 0.1) (type default)) (fill none) (layer "Edge.Cuts"))
 (segment (start 76.135 46.355) (end 85.185 46.355) (width 0.25) (layer "F.Cu") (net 4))
 (segment (start 76.135 46.355) (end 75.160001 46.355) (width 0.25) (layer "F.Cu") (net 4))
 (segment (start 85.185 46.355) (end 86.36 45.18) (width 0.25) (layer "F.Cu") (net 4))
 (segment (start 73.890001 45.085) (end 71.185 45.085) (width 0.25) (layer "F.Cu") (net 4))
 (segment (start 86.36 45.18) (end 86.36 58.42) (width 0.25) (layer "F.Cu") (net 4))
 (segment (start 75.160001 46.355) (end 73.890001 45.085) (width 0.25) (layer "F.Cu") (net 4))
 (segment (start 76.16 35.56) (end 76.2 35.56) (width 0.25) (layer "F.Cu") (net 1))
 (via (at 81.28 38.1) (size 0.8) (drill 0.4) (layers "F.Cu" "B.Cu") (free) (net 1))
 (via (at 91.44 38.1) (size 0.8) (drill 0.4) (layers "F.Cu" "B.Cu") (free) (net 1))
 (segment (start 81.28 38.1) (end 91.44 38.1) (width 0.5) (layer "B.Cu") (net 1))
 (segment (start 76.2 47.69) (end 76.135 47.625) (width 0.25) (layer "F.Cu") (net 8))
 (segment (start 76.2 57.3825) (end 76.2 47.69) (width 0.25) (layer "F.Cu") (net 8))
 (segment (start 63.5 35.56) (end 63.5 43.18) (width 0.25) (layer "F.Cu") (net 6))
 (segment (start 70.685 32.585) (end 73.66 35.56) (width 0.5) (layer "F.Cu") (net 5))
 (segment (start 84.82 32.02) (end 77.2 32.02) (width 0.5) (layer "F.Cu") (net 5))
 (segment (start 73.66 35.56) (end 73.66 41.34) (width 0.5) (layer "F.Cu") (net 5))
 (segment (start 76.135 43.815) (end 78.105 43.815) (width 0.5) (layer "F.Cu") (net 5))
 (segment (start 71.185 53.275) (end 71.185 47.625) (width 0.5) (layer "F.Cu") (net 5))
 (segment (start 63.5 32.585) (end 70.685 32.585) (width 0.5) (layer "F.Cu") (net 5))
 (segment (start 84.82 32.02) (end 84.82 32.223122) (width 0.5) (layer "F.Cu") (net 5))
 (segment (start 71.185 53.405) (end 71.12 53.34) (width 0.5) (layer "F.Cu") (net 5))
 (segment (start 71.12 53.34) (end 71.185 53.275) (width 0.5) (layer "F.Cu") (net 5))
 (segment (start 73.66 41.34) (end 76.135 43.815) (width 0.5) (layer "F.Cu") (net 5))
 (segment (start 77.2 32.02) (end 73.66 35.56) (width 0.5) (layer "F.Cu") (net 5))
 (segment (start 78.105 43.815) (end 81.28 40.64) (width 0.5) (layer "F.Cu") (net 5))
 (via (at 71.12 53.34) (size 0.8) (drill 0.4) (layers "F.Cu" "B.Cu") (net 5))
 (via (at 81.28 40.64) (size 0.8) (drill 0.4) (layers "F.Cu" "B.Cu") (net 5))
 (segment (start 78.74 53.34) (end 81.28 50.8) (width 0.5) (layer "B.Cu") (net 5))
 (segment (start 71.12 53.34) (end 78.74 53.34) (width 0.5) (layer "B.Cu") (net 5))
 (segment (start 81.28 50.8) (end 81.28 40.64) (width 0.5) (layer "B.Cu") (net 5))
 (segment (start 63.5 52.8) (end 63.5 57.3675) (width 0.25) (layer "F.Cu") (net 2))
 (segment (start 63.5 57.3675) (end 64.5525 58.42) (width 0.25) (layer "F.Cu") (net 2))
 (segment (start 86.36 43.18) (end 84.455 45.085) (width 0.25) (layer "F.Cu") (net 3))
 (segment (start 84.455 45.085) (end 76.135 45.085) (width 0.25) (layer "F.Cu") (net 3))
 (segment (start 84.82 34.02) (end 84.82 41.64) (width 0.25) (layer "F.Cu") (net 3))
 (segment (start 84.82 41.64) (end 86.36 43.18) (width 0.25) (layer "F.Cu") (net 3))
 (segment (start 63.5 45.18) (end 64.675 46.355) (width 0.25) (layer "F.Cu") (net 7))
 (segment (start 63.5 45.18) (end 63.5 50.8) (width 0.25) (layer "F.Cu") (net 7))
 (segment (start 64.675 46.355) (end 71.185 46.355) (width 0.25) (layer "F.Cu") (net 7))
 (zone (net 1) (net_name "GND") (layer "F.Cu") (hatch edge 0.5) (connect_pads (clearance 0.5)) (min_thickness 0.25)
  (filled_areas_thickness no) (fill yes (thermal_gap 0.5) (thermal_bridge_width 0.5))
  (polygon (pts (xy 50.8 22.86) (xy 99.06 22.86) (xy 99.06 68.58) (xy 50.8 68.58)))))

